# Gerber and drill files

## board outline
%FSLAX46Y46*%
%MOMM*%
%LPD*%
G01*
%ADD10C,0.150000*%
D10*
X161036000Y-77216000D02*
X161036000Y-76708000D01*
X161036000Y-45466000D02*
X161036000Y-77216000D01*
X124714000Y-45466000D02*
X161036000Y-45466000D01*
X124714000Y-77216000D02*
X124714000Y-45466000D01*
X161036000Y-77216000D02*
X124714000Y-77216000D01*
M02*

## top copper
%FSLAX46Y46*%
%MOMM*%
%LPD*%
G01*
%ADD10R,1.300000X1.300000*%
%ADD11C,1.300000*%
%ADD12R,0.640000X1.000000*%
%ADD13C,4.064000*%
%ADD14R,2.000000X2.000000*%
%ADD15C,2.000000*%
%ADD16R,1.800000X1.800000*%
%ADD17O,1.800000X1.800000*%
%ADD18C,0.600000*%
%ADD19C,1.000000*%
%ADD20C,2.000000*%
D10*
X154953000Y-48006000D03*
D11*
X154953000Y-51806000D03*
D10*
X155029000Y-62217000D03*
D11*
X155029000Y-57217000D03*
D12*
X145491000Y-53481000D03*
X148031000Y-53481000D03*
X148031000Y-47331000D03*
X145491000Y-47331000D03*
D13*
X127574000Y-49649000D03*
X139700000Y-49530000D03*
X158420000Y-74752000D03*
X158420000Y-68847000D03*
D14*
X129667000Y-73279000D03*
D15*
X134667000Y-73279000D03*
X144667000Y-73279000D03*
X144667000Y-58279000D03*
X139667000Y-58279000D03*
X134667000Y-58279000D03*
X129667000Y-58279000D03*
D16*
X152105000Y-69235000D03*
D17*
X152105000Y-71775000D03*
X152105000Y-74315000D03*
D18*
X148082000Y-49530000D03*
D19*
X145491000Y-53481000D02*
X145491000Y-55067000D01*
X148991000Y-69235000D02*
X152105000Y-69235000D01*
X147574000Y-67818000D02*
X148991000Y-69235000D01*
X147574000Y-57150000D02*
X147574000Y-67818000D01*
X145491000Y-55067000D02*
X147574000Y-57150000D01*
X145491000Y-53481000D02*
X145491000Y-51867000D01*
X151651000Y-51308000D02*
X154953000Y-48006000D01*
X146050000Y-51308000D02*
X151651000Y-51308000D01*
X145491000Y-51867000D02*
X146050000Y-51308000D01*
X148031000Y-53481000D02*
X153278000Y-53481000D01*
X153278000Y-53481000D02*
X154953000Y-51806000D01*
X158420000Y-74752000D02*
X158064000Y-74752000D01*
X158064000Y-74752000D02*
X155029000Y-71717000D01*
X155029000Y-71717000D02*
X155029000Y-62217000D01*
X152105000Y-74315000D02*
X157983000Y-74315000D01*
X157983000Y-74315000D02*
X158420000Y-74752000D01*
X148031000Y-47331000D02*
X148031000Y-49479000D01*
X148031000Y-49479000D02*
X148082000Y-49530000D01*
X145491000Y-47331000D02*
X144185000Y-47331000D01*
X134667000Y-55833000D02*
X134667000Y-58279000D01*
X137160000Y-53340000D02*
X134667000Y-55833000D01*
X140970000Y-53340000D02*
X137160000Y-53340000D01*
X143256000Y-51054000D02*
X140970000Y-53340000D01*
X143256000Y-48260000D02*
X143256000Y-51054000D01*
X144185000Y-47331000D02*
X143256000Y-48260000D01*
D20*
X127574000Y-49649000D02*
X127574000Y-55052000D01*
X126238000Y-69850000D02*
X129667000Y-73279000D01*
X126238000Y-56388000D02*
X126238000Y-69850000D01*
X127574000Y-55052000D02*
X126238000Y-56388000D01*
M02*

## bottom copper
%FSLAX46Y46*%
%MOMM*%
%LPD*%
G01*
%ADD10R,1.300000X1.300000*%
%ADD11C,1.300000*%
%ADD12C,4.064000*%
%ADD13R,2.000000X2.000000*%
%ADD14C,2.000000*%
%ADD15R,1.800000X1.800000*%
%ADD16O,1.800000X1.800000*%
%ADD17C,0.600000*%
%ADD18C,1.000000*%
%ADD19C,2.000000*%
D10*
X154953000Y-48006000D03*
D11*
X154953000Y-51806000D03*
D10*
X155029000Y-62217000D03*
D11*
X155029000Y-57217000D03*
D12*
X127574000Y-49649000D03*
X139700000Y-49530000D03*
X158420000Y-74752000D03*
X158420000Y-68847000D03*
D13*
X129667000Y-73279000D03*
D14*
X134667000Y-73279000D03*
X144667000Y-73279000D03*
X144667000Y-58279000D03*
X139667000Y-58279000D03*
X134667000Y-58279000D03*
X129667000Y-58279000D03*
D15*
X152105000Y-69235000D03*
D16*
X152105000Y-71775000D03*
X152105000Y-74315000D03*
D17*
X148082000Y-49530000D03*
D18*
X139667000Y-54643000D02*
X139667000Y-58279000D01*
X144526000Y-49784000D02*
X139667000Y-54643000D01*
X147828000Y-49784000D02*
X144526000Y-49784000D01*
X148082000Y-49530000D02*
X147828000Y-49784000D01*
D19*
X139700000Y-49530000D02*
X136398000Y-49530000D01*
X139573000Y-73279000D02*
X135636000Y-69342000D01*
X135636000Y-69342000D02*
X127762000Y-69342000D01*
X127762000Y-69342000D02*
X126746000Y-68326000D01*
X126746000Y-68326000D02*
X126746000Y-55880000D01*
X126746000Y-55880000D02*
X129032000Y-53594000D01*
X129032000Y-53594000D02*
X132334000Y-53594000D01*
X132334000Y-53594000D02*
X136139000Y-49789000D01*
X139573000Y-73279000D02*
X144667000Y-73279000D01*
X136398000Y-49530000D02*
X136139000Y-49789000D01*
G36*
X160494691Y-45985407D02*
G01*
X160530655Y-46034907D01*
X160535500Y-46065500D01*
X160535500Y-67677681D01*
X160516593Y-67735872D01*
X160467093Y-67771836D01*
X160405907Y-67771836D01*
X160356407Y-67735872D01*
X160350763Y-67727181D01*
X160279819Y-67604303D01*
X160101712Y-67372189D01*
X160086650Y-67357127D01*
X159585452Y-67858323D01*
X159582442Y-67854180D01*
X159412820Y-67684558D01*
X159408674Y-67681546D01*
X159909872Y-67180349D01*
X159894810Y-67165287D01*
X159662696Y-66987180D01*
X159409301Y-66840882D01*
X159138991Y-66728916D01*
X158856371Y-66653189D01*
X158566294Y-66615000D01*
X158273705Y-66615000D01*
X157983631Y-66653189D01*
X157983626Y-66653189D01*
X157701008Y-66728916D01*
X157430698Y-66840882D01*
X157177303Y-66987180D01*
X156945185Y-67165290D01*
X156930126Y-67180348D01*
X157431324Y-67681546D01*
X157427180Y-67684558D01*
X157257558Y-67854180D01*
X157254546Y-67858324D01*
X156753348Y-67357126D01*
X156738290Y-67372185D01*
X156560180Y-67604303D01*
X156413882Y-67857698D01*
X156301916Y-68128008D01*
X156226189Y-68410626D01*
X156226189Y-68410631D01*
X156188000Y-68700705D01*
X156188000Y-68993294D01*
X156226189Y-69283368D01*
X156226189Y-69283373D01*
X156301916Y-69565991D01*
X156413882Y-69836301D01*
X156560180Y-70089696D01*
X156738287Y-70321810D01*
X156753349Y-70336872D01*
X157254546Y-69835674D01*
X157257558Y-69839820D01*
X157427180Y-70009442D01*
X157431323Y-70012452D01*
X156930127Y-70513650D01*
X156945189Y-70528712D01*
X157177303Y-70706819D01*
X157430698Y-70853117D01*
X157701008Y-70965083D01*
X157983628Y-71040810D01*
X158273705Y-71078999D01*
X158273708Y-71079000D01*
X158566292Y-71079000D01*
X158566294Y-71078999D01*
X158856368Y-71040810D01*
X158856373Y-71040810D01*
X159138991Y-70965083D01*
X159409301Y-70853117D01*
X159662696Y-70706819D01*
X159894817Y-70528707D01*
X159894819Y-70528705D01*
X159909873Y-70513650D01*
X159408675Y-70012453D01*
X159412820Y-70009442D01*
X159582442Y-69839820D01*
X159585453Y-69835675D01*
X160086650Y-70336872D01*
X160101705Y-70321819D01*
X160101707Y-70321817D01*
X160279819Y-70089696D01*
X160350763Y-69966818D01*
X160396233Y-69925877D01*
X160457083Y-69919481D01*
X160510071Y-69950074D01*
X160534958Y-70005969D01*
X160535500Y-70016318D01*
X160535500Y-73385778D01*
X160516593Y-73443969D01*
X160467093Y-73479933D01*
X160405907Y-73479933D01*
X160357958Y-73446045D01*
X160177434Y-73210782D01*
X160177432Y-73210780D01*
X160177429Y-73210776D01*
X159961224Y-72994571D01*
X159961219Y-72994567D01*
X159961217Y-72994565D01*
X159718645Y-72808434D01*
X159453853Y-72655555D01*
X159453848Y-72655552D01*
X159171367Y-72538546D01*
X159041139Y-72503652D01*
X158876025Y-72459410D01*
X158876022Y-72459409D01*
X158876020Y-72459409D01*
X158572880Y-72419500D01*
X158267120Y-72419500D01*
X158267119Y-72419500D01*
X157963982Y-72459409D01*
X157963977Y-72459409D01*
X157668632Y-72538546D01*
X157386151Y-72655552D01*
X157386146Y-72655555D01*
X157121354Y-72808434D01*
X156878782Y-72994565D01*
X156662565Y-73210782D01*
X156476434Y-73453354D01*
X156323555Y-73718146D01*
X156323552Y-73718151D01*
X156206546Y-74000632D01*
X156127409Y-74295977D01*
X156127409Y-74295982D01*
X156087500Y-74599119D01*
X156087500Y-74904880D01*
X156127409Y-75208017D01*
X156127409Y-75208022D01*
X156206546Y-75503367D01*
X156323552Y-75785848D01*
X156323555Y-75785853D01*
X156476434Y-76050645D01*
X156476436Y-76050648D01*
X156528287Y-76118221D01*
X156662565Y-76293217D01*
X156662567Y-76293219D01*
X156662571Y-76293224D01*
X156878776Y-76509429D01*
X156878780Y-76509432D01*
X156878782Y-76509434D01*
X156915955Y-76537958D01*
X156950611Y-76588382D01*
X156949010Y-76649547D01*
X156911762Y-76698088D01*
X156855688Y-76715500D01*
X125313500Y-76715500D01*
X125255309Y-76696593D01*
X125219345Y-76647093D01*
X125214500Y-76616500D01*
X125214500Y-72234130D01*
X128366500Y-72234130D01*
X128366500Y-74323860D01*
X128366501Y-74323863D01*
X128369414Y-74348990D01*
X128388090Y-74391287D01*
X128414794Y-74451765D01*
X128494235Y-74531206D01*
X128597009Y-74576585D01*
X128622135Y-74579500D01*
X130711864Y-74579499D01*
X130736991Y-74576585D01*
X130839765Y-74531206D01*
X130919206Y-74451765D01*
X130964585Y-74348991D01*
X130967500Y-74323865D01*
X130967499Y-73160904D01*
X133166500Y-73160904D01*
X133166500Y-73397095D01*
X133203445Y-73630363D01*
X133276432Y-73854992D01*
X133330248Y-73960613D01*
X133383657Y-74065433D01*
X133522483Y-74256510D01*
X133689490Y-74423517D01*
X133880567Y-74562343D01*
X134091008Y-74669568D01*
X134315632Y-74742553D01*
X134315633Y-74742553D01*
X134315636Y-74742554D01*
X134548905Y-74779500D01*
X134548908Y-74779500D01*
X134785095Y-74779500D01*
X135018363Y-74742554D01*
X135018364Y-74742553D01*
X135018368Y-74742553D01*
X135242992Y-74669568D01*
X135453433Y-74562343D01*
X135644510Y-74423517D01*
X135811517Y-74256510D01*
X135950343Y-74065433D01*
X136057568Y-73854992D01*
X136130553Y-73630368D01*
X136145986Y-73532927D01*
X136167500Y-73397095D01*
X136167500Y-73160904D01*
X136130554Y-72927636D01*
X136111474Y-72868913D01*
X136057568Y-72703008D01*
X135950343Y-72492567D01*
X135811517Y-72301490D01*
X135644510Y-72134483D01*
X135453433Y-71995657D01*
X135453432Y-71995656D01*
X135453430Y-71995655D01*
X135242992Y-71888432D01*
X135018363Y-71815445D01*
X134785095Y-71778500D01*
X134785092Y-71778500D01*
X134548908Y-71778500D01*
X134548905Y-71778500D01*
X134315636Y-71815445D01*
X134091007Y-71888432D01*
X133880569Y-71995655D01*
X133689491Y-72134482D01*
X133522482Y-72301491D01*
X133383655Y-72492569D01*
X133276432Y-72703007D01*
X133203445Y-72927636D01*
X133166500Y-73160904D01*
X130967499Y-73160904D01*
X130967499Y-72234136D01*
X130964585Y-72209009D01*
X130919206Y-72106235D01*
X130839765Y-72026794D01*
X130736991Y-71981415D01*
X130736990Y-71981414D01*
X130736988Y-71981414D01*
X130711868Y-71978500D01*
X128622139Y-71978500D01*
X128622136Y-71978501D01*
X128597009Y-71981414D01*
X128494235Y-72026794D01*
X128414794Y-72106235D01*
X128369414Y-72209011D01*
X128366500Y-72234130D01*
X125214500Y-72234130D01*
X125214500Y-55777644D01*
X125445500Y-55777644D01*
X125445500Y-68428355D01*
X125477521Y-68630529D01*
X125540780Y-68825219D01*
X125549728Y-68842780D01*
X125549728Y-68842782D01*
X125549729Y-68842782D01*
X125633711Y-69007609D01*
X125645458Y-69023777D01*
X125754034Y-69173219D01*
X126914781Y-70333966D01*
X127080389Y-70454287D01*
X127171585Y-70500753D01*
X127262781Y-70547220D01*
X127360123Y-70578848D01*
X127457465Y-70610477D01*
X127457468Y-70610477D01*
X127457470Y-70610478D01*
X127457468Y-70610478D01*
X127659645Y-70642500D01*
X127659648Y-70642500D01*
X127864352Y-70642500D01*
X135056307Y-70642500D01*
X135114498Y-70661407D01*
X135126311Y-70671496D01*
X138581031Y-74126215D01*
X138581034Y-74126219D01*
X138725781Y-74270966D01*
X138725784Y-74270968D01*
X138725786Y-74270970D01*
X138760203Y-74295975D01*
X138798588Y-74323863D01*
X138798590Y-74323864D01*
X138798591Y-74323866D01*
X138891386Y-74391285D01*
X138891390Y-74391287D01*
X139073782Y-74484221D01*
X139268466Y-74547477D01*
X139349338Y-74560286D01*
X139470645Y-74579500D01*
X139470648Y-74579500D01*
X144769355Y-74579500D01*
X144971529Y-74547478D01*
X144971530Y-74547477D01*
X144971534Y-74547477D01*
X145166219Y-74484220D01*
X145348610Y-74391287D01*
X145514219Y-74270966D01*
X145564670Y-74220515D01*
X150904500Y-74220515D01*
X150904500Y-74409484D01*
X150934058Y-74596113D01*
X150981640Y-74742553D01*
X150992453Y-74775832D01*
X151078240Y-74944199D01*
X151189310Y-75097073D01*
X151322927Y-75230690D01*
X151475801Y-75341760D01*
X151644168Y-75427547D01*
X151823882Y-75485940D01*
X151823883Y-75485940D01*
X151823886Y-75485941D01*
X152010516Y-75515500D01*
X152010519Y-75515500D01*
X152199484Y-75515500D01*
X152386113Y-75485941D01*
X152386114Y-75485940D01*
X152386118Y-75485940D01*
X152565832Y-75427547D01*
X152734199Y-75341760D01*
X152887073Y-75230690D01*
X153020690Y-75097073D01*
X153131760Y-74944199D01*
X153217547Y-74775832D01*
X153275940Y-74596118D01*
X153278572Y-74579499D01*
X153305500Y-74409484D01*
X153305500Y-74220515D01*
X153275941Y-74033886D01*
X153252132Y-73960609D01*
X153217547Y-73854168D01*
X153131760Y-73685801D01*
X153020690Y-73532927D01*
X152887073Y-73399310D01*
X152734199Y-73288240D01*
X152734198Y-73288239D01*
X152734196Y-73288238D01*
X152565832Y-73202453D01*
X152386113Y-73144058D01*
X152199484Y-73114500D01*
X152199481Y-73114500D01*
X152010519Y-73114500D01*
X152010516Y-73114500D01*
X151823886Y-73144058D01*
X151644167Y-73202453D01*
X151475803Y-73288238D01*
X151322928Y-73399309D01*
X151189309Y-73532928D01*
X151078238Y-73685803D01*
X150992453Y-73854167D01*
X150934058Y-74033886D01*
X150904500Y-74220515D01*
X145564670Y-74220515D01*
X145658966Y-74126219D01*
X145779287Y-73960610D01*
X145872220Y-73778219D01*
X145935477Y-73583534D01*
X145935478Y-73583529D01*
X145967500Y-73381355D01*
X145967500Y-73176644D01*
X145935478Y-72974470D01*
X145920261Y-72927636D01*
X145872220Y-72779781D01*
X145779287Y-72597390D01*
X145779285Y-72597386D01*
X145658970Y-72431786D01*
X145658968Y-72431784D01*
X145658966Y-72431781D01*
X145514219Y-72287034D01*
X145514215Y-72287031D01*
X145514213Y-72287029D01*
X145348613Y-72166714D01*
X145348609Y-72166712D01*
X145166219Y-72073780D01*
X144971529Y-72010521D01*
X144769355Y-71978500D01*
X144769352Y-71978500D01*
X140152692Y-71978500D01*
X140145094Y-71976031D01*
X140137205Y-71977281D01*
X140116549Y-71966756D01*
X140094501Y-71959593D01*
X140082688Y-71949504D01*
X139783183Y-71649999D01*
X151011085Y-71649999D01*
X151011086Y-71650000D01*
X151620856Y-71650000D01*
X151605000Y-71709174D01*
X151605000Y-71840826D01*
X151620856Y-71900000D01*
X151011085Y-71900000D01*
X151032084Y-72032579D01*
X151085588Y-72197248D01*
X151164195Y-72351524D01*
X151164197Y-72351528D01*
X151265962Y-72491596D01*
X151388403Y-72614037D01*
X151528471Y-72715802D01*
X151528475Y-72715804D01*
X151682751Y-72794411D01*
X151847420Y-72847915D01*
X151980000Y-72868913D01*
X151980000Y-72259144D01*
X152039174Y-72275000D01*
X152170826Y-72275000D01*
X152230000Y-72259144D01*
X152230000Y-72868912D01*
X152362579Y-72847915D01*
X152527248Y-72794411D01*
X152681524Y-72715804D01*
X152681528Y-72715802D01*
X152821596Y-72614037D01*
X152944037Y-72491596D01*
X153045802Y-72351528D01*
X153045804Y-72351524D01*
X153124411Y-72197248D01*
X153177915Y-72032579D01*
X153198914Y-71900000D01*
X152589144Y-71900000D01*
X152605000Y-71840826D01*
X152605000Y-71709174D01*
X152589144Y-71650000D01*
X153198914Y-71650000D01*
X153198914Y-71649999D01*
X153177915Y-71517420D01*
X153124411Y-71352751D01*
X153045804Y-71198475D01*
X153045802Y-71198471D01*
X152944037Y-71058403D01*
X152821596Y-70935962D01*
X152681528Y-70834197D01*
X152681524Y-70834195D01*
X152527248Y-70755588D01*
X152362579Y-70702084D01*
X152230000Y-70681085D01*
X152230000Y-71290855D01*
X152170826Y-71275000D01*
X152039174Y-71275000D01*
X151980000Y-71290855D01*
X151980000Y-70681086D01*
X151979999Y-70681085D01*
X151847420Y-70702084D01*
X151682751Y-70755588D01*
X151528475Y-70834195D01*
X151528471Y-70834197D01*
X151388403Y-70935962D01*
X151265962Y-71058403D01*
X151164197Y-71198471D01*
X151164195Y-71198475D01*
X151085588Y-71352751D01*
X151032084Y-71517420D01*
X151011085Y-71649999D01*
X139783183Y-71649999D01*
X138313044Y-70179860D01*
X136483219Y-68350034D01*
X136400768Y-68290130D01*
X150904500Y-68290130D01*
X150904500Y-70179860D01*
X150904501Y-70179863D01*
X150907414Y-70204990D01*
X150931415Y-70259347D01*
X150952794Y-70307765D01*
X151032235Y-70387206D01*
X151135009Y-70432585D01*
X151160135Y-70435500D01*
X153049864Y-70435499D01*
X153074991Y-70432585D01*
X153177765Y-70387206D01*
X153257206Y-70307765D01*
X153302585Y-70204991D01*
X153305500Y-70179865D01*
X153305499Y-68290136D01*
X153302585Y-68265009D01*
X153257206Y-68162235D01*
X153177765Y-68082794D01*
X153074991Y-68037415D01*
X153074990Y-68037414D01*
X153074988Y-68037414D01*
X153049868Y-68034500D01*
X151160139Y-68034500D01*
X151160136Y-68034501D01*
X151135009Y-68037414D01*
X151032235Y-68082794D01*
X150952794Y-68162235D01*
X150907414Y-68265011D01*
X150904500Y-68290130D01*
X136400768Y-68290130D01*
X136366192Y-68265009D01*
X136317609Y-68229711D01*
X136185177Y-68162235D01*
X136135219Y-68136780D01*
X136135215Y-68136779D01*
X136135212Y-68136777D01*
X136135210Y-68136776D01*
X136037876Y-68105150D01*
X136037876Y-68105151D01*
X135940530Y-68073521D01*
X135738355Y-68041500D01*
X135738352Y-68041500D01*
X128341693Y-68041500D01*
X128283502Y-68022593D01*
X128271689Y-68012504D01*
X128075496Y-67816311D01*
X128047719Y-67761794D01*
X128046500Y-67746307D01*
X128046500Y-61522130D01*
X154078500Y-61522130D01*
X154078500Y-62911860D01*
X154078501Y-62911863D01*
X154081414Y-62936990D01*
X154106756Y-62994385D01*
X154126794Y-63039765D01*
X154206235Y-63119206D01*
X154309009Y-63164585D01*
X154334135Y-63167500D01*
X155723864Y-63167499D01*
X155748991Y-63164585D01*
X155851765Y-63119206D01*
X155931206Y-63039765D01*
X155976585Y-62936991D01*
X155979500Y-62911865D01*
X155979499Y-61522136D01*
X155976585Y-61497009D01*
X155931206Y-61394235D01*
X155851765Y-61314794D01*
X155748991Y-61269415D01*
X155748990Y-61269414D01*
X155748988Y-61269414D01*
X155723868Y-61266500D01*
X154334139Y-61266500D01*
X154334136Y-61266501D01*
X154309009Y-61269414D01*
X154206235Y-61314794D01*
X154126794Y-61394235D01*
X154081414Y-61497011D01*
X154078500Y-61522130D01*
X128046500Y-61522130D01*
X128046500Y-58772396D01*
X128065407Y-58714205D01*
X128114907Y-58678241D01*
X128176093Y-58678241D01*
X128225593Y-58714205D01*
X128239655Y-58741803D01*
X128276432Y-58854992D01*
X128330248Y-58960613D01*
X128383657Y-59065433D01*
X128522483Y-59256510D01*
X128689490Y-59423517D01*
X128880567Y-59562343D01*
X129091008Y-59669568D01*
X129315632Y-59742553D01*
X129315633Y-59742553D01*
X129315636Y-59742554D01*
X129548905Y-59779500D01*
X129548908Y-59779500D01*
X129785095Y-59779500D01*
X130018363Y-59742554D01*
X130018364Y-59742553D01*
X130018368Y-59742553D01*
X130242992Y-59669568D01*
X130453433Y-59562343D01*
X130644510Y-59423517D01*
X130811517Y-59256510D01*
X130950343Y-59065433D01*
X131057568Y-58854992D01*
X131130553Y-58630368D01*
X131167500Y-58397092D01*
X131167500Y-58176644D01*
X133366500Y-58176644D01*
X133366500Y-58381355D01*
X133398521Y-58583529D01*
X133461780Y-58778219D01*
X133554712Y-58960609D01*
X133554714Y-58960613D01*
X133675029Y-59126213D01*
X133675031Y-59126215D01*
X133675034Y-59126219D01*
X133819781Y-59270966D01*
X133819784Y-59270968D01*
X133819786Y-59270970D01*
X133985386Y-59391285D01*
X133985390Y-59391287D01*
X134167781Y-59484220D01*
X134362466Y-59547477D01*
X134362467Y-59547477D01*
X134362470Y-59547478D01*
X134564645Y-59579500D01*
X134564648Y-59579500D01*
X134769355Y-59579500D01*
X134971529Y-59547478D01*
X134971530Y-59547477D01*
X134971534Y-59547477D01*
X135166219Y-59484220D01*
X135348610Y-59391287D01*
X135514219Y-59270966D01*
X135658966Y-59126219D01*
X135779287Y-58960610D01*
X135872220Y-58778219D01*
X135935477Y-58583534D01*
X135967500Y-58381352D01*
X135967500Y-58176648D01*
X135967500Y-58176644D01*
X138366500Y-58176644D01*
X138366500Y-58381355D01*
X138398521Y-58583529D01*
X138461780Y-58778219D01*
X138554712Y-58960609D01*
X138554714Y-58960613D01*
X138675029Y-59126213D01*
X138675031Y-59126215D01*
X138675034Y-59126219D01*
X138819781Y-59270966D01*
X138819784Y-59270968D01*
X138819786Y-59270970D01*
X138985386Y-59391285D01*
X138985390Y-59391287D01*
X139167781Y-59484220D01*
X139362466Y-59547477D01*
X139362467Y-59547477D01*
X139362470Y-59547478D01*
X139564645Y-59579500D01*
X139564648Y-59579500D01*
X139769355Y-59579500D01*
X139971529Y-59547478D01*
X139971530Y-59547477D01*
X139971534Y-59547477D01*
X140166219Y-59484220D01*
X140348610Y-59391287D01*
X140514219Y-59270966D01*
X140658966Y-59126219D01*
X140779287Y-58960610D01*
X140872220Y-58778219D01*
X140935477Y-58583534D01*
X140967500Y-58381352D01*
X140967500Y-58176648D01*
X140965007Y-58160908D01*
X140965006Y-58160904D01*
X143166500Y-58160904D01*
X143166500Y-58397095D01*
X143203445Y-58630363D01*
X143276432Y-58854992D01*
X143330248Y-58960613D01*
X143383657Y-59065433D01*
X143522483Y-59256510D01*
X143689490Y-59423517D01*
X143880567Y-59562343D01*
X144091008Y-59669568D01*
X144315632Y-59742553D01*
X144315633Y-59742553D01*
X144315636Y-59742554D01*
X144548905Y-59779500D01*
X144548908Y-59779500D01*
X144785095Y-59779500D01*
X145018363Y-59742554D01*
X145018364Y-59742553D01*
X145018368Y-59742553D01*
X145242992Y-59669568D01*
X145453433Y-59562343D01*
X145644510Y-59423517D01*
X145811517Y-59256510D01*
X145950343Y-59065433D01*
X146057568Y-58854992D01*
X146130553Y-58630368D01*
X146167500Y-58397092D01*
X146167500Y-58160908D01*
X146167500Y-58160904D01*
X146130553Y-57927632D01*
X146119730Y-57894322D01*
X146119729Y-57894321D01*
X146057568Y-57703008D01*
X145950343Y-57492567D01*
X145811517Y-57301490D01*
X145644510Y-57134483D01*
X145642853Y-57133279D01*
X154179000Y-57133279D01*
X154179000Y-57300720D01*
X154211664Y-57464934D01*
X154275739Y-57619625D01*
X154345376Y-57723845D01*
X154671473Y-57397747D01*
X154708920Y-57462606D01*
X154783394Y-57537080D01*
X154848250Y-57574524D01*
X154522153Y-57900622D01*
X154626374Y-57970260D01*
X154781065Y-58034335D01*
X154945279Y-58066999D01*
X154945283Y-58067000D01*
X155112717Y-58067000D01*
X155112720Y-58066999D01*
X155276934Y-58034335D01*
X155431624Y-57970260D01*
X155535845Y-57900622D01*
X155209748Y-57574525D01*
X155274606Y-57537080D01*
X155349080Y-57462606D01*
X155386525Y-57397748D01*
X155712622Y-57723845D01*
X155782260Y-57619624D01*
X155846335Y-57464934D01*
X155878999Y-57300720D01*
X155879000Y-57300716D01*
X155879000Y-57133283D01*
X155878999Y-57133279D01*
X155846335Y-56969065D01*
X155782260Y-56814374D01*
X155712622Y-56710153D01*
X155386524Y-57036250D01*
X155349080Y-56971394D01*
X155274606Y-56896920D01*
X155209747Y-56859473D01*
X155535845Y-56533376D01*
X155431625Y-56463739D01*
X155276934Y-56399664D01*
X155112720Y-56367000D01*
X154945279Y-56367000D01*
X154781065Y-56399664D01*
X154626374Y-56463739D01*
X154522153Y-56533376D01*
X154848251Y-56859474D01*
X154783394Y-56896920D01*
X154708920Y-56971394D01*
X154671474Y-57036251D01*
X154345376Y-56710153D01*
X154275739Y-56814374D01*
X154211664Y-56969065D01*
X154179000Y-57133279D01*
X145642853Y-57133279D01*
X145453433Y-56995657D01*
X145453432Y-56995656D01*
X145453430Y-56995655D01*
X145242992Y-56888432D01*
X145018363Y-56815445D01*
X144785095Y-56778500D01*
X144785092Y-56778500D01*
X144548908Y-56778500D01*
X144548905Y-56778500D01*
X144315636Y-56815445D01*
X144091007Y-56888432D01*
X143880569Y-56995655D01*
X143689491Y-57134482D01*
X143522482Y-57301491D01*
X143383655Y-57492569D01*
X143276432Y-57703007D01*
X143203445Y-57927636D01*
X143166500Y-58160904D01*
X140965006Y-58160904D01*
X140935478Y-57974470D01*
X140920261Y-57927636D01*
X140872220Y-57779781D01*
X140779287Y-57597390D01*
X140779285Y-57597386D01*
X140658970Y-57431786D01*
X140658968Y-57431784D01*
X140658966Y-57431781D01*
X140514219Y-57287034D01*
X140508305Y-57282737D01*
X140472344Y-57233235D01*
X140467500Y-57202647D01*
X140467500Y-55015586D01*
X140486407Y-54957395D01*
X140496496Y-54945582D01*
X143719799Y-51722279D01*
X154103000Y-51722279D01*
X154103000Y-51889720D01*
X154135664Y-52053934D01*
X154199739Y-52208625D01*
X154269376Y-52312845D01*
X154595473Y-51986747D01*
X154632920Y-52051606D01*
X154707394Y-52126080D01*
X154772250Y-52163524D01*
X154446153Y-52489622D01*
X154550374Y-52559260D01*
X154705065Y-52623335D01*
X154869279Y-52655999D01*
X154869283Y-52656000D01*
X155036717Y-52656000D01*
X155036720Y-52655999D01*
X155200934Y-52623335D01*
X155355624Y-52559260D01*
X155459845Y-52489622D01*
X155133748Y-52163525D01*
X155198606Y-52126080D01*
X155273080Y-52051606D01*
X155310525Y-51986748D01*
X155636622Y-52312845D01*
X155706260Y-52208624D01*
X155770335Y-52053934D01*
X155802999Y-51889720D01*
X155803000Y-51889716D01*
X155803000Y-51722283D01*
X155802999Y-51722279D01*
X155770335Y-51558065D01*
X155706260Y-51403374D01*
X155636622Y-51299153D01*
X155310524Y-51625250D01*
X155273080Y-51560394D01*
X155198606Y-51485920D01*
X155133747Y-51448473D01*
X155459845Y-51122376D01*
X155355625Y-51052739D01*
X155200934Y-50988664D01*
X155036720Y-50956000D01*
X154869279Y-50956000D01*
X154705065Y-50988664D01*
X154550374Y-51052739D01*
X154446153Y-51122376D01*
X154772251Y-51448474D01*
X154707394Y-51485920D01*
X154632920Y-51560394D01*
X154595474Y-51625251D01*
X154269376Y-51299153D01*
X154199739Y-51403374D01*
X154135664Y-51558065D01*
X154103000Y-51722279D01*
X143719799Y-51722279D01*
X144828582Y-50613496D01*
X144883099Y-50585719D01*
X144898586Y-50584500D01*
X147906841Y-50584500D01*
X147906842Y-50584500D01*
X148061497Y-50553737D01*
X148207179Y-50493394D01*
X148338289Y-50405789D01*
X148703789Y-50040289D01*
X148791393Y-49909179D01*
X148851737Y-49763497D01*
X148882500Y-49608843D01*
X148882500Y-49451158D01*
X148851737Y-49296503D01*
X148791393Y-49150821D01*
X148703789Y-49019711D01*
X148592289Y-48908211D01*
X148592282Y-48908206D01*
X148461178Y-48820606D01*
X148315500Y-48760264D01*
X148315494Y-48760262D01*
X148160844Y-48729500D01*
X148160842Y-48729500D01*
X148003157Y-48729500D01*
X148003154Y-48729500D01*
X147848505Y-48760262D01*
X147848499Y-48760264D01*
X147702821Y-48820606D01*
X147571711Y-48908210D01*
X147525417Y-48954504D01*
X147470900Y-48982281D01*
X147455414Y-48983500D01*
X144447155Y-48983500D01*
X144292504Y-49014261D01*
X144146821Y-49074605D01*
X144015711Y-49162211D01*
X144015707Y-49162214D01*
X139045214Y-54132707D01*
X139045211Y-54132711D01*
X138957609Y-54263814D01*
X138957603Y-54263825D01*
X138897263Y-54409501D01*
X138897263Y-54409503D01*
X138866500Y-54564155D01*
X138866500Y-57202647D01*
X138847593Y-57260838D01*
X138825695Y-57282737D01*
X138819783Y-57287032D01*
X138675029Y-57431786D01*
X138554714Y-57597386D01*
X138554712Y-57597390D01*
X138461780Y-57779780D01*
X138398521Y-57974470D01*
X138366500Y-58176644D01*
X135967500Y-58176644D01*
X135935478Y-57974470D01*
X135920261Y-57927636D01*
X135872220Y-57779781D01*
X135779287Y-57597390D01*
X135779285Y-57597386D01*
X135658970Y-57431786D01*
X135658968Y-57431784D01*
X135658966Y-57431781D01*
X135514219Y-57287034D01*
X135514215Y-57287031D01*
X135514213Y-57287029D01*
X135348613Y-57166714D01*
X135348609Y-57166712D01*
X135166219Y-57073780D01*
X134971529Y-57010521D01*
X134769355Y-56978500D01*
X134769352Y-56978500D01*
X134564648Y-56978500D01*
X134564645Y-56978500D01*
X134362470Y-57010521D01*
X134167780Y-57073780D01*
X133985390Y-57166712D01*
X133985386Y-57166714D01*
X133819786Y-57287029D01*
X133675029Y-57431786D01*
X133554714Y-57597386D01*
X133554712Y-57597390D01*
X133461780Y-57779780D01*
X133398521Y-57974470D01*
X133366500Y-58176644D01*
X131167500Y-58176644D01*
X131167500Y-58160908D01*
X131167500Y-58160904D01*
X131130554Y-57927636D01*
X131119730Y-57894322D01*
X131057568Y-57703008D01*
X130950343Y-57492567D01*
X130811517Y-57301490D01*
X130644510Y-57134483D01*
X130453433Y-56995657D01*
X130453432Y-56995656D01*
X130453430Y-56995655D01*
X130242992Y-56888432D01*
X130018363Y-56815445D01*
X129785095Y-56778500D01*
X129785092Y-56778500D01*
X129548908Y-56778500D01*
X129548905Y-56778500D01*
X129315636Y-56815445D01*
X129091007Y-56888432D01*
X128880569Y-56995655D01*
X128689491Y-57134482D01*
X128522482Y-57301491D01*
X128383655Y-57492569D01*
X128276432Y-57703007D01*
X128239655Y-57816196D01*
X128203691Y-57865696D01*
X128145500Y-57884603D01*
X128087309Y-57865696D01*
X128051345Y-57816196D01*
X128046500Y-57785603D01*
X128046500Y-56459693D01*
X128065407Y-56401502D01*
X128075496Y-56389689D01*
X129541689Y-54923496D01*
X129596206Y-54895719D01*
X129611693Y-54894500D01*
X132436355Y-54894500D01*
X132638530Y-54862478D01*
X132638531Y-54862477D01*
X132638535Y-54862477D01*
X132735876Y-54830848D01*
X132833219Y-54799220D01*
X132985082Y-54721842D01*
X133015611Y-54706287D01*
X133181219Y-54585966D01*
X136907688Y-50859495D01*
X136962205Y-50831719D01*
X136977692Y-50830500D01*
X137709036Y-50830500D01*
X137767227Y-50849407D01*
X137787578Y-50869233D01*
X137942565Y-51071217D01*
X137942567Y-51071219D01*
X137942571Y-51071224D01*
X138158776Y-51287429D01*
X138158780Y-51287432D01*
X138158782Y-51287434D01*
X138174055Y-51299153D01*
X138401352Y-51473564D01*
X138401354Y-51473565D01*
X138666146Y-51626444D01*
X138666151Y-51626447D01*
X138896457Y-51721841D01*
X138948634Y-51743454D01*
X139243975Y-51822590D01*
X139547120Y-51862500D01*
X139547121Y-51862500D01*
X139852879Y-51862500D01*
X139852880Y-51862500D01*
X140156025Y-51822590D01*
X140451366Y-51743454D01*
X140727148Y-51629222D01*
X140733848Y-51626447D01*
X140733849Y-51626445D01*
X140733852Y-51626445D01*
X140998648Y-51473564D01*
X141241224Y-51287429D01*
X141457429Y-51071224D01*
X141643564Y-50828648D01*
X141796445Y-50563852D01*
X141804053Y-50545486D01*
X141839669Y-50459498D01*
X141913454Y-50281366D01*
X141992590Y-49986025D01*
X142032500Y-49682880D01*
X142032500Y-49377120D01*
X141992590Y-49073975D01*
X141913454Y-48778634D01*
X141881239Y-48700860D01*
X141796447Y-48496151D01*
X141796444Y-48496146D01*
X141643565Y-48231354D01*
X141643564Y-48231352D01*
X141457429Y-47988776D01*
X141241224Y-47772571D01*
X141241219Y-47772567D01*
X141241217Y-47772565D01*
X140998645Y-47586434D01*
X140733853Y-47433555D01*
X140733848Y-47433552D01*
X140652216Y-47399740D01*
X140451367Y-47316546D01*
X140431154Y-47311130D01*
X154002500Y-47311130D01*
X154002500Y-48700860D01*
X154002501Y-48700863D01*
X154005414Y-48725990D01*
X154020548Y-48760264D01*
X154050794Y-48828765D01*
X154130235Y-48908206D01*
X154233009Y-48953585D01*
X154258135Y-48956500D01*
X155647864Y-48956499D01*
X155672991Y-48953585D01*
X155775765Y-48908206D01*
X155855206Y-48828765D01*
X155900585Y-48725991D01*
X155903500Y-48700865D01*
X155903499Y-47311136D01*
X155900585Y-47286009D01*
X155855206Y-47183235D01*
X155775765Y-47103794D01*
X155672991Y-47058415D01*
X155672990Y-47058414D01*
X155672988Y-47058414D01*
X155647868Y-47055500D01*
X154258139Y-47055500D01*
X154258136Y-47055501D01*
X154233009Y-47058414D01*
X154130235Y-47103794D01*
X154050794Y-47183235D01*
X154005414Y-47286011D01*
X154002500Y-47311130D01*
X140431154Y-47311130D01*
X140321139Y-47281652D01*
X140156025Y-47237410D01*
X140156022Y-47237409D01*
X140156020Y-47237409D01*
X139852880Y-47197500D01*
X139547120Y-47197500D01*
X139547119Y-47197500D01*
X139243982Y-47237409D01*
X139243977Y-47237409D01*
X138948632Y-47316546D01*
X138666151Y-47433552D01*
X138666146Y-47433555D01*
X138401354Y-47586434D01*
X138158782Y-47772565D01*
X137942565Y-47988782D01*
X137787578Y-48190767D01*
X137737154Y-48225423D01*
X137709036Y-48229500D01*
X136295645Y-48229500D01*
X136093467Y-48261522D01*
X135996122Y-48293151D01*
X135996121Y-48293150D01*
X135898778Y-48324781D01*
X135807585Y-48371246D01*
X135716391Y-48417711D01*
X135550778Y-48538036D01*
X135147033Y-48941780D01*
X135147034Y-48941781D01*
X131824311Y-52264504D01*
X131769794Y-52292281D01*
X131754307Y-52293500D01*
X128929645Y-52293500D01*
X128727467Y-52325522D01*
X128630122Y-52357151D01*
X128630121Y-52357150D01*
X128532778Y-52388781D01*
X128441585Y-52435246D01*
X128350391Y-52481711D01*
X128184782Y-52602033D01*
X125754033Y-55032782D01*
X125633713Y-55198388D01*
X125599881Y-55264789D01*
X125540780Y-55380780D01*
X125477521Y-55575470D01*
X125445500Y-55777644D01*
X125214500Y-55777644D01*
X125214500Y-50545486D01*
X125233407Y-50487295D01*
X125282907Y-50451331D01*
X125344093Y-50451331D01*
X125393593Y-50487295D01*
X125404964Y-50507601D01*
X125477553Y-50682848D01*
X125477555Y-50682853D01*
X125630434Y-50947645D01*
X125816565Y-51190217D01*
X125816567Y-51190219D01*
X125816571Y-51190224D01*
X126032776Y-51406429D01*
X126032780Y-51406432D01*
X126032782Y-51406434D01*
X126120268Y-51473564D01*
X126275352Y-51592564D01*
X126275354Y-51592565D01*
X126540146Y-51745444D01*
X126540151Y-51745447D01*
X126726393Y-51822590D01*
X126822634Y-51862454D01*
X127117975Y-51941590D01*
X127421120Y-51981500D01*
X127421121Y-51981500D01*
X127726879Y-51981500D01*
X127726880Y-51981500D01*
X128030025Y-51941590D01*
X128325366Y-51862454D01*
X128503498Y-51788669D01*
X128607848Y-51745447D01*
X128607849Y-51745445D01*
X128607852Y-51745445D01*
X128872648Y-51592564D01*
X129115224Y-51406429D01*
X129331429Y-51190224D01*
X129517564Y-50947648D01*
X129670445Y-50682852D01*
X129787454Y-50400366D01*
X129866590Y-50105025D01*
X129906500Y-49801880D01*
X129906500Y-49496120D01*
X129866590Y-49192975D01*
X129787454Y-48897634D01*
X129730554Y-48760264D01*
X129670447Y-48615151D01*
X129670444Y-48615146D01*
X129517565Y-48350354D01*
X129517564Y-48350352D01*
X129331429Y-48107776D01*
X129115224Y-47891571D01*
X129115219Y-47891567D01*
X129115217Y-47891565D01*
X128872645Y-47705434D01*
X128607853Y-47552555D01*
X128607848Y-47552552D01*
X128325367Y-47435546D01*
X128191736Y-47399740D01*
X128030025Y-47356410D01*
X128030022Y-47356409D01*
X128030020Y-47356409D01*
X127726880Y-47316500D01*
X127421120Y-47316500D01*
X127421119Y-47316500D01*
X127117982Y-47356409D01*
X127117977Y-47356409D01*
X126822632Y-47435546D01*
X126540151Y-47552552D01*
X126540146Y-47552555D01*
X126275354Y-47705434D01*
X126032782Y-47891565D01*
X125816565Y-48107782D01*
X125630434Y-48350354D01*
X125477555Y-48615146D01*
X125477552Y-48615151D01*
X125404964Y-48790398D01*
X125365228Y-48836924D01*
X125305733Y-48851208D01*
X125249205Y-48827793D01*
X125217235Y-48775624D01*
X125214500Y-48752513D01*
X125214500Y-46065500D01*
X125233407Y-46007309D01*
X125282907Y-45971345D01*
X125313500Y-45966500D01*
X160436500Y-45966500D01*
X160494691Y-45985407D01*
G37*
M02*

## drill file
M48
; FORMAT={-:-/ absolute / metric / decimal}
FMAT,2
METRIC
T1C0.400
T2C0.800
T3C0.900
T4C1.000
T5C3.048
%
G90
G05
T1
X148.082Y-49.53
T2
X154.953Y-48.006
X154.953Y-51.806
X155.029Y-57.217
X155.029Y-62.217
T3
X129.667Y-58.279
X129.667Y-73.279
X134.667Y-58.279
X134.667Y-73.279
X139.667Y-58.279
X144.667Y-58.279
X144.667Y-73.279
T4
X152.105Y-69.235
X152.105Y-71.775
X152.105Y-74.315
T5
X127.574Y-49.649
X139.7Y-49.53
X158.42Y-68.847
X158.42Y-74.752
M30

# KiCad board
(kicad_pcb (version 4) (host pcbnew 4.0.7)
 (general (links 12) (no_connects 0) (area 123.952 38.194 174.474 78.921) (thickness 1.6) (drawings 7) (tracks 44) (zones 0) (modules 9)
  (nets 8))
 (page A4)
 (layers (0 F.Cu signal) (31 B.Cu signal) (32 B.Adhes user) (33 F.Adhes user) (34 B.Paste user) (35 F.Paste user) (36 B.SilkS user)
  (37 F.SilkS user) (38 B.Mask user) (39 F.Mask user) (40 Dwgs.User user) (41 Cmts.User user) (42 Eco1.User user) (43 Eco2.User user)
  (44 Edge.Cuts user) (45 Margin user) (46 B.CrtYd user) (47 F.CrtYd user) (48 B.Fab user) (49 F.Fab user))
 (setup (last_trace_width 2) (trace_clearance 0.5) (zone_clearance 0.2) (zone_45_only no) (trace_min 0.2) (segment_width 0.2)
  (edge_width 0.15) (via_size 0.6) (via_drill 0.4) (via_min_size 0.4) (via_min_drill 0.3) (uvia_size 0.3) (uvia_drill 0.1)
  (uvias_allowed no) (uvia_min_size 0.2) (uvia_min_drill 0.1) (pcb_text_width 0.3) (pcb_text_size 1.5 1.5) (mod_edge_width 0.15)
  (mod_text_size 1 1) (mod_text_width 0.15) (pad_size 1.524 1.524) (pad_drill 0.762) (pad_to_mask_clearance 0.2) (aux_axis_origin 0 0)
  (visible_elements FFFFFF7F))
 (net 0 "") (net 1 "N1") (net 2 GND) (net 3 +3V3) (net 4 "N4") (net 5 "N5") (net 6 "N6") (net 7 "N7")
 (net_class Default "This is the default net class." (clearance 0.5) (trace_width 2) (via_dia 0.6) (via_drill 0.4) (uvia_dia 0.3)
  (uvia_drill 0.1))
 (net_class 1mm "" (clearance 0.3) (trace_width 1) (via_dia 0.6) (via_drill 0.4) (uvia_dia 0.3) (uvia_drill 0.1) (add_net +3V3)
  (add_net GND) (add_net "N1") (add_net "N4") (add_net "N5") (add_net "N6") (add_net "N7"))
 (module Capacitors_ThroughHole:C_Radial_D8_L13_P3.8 (layer F.Cu) (at 154.953 48.006 270)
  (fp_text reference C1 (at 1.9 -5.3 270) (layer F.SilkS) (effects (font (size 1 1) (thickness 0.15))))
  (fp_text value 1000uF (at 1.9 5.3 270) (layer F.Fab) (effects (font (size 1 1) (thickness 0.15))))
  (pad 1 thru_hole rect (at 0 0 270) (size 1.3 1.3) (drill 0.8) (layers *.Cu *.Mask) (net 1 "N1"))
  (pad 2 thru_hole circle (at 3.8 0 270) (size 1.3 1.3) (drill 0.8) (layers *.Cu *.Mask) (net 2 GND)))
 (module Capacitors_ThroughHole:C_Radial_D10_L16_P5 (layer F.Cu) (at 155.029 62.217 90)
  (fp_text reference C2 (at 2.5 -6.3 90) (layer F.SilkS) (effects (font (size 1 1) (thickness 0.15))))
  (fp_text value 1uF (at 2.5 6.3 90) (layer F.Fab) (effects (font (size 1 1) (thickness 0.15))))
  (pad 1 thru_hole rect (at 0 0 90) (size 1.3 1.3) (drill 0.8) (layers *.Cu *.Mask) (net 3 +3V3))
  (pad 2 thru_hole circle (at 5 0 90) (size 1.3 1.3) (drill 0.8) (layers *.Cu *.Mask) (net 2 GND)))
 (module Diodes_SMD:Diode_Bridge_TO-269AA (layer F.Cu) (at 146.761 50.406 90)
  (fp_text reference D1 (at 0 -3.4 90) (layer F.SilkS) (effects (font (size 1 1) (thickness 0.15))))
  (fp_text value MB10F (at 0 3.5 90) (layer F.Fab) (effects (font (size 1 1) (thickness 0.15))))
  (pad 1 smd rect (at -3.075 -1.27 90) (size 1 0.64) (layers F.Cu F.Paste F.Mask) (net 1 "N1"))
  (pad 2 smd rect (at -3.075 1.27 90) (size 1 0.64) (layers F.Cu F.Paste F.Mask) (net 2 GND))
  (pad 3 smd rect (at 3.075 1.27 90) (size 1 0.64) (layers F.Cu F.Paste F.Mask) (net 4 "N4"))
  (pad 4 smd rect (at 3.075 -1.27 90) (size 1 0.64) (layers F.Cu F.Paste F.Mask) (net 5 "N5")))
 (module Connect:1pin (layer F.Cu) (at 127.574 49.649)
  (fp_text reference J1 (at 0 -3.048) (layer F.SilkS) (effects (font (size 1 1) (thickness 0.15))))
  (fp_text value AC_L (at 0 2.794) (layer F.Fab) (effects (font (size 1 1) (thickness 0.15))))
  (pad 1 thru_hole circle (at 0 0) (size 4.064 4.064) (drill 3.048) (layers *.Cu *.Mask) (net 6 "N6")))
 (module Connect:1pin (layer F.Cu) (at 139.7 49.53)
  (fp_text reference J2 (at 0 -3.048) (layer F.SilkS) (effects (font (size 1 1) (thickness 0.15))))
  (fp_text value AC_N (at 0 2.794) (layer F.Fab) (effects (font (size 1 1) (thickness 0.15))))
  (pad 1 thru_hole circle (at 0 0) (size 4.064 4.064) (drill 3.048) (layers *.Cu *.Mask) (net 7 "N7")))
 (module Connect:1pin (layer F.Cu) (at 158.42 74.752)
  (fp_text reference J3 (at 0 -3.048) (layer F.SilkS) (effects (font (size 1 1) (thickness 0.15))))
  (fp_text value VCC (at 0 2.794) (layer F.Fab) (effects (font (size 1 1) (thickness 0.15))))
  (pad 1 thru_hole circle (at 0 0) (size 4.064 4.064) (drill 3.048) (layers *.Cu *.Mask) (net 3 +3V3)))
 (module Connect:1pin (layer F.Cu) (at 158.42 68.847)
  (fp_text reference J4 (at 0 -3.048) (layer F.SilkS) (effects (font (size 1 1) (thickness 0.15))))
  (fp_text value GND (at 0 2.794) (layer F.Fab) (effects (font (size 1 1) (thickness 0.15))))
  (pad 1 thru_hole circle (at 0 0) (size 4.064 4.064) (drill 3.048) (layers *.Cu *.Mask) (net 2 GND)))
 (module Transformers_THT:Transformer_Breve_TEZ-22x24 (layer F.Cu) (at 129.667 73.279)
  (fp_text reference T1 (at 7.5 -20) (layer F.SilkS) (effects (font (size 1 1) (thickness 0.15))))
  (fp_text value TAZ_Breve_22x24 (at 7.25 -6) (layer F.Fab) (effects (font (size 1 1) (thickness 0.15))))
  (pad 1 thru_hole rect (at 0 0) (size 2 2) (drill 0.9) (layers *.Cu *.Mask) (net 6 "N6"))
  (pad 2 thru_hole circle (at 5 0) (size 2 2) (drill 0.9) (layers *.Cu *.Mask))
  (pad 4 thru_hole circle (at 15 0) (size 2 2) (drill 0.9) (layers *.Cu *.Mask) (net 7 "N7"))
  (pad 5 thru_hole circle (at 15 -15) (size 2 2) (drill 0.9) (layers *.Cu *.Mask))
  (pad 6 thru_hole circle (at 10 -15) (size 2 2) (drill 0.9) (layers *.Cu *.Mask) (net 4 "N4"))
  (pad 7 thru_hole circle (at 5 -15) (size 2 2) (drill 0.9) (layers *.Cu *.Mask) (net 5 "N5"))
  (pad 8 thru_hole circle (at 0 -15) (size 2 2) (drill 0.9) (layers *.Cu *.Mask)))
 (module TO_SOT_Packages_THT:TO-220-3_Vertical (layer F.Cu) (at 152.105 69.235 270)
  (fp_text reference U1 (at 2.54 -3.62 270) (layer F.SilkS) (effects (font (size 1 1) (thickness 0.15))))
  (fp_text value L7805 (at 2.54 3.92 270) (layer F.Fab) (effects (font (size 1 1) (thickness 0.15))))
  (pad 1 thru_hole rect (at 0 0 270) (size 1.8 1.8) (drill 1) (layers *.Cu *.Mask) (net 1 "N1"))
  (pad 2 thru_hole oval (at 2.54 0 270) (size 1.8 1.8) (drill 1) (layers *.Cu *.Mask) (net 2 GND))
  (pad 3 thru_hole oval (at 5.08 0 270) (size 1.8 1.8) (drill 1) (layers *.Cu *.Mask) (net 3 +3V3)))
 (gr_line (start 161.036 77.216) (end 161.036 76.708) (angle 90) (layer Edge.Cuts) (width 0.15))
 (gr_line (start 161.036 45.466) (end 161.036 77.216) (angle 90) (layer Edge.Cuts) (width 0.15))
 (gr_line (start 124.714 45.466) (end 161.036 45.466) (angle 90) (layer Edge.Cuts) (width 0.15))
 (gr_line (start 124.714 77.216) (end 124.714 45.466) (angle 90) (layer Edge.Cuts) (width 0.15))
 (gr_line (start 161.036 77.216) (end 124.714 77.216) (angle 90) (layer Edge.Cuts) (width 0.15))
 (segment (start 145.491 53.481) (end 145.491 55.067) (width 1) (layer F.Cu) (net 1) (status 400000))
 (segment (start 148.991 69.235) (end 152.105 69.235) (width 1) (layer F.Cu) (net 1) (status 800000))
 (segment (start 147.574 67.818) (end 148.991 69.235) (width 1) (layer F.Cu) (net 1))
 (segment (start 147.574 57.15) (end 147.574 67.818) (width 1) (layer F.Cu) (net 1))
 (segment (start 145.491 55.067) (end 147.574 57.15) (width 1) (layer F.Cu) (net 1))
 (segment (start 145.491 53.481) (end 145.491 51.867) (width 1) (layer F.Cu) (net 1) (status 400000))
 (segment (start 151.651 51.308) (end 154.953 48.006) (width 1) (layer F.Cu) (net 1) (status 800000))
 (segment (start 146.05 51.308) (end 151.651 51.308) (width 1) (layer F.Cu) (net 1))
 (segment (start 145.491 51.867) (end 146.05 51.308) (width 1) (layer F.Cu) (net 1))
 (segment (start 148.031 53.481) (end 153.278 53.481) (width 1) (layer F.Cu) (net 2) (status 400000))
 (segment (start 153.278 53.481) (end 154.953 51.806) (width 1) (layer F.Cu) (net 2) (status 800000))
 (segment (start 158.42 74.752) (end 158.064 74.752) (width 1) (layer F.Cu) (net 3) (status C00000))
 (segment (start 158.064 74.752) (end 155.029 71.717) (width 1) (layer F.Cu) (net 3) (status 400000))
 (segment (start 155.029 71.717) (end 155.029 62.217) (width 1) (layer F.Cu) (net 3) (status 800000))
 (segment (start 152.105 74.315) (end 157.983 74.315) (width 1) (layer F.Cu) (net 3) (status C00000))
 (segment (start 157.983 74.315) (end 158.42 74.752) (width 1) (layer F.Cu) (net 3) (status C00000))
 (segment (start 148.031 47.331) (end 148.031 49.479) (width 1) (layer F.Cu) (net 4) (status 400000))
 (segment (start 139.667 54.643) (end 139.667 58.279) (width 1) (layer B.Cu) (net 4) (status 800000))
 (segment (start 144.526 49.784) (end 139.667 54.643) (width 1) (layer B.Cu) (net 4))
 (segment (start 147.828 49.784) (end 144.526 49.784) (width 1) (layer B.Cu) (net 4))
 (segment (start 148.082 49.53) (end 147.828 49.784) (width 1) (layer B.Cu) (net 4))
 (via (at 148.082 49.53) (size 0.6) (drill 0.4) (layers F.Cu B.Cu) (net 4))
 (segment (start 148.031 49.479) (end 148.082 49.53) (width 1) (layer F.Cu) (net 4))
 (segment (start 145.491 47.331) (end 144.185 47.331) (width 1) (layer F.Cu) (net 5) (status 400000))
 (segment (start 134.667 55.833) (end 134.667 58.279) (width 1) (layer F.Cu) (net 5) (status 800000))
 (segment (start 137.16 53.34) (end 134.667 55.833) (width 1) (layer F.Cu) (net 5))
 (segment (start 140.97 53.34) (end 137.16 53.34) (width 1) (layer F.Cu) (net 5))
 (segment (start 143.256 51.054) (end 140.97 53.34) (width 1) (layer F.Cu) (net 5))
 (segment (start 143.256 48.26) (end 143.256 51.054) (width 1) (layer F.Cu) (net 5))
 (segment (start 144.185 47.331) (end 143.256 48.26) (width 1) (layer F.Cu) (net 5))
 (segment (start 127.574 49.649) (end 127.574 55.052) (width 2) (layer F.Cu) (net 6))
 (segment (start 126.238 69.85) (end 129.667 73.279) (width 2) (layer F.Cu) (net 6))
 (segment (start 126.238 56.388) (end 126.238 69.85) (width 2) (layer F.Cu) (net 6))
 (segment (start 127.574 55.052) (end 126.238 56.388) (width 2) (layer F.Cu) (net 6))
 (segment (start 139.7 49.53) (end 136.398 49.53) (width 2) (layer B.Cu) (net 7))
 (segment (start 139.573 73.279) (end 135.636 69.342) (width 2) (layer B.Cu) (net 7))
 (segment (start 135.636 69.342) (end 127.762 69.342) (width 2) (layer B.Cu) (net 7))
 (segment (start 127.762 69.342) (end 126.746 68.326) (width 2) (layer B.Cu) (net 7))
 (segment (start 126.746 68.326) (end 126.746 55.88) (width 2) (layer B.Cu) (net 7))
 (segment (start 126.746 55.88) (end 129.032 53.594) (width 2) (layer B.Cu) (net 7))
 (segment (start 129.032 53.594) (end 132.334 53.594) (width 2) (layer B.Cu) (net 7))
 (segment (start 132.334 53.594) (end 136.139 49.789) (width 2) (layer B.Cu) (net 7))
 (segment (start 139.573 73.279) (end 144.667 73.279) (width 2) (layer B.Cu) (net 7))
 (segment (start 136.398 49.53) (end 136.139 49.789) (width 2) (layer B.Cu) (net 7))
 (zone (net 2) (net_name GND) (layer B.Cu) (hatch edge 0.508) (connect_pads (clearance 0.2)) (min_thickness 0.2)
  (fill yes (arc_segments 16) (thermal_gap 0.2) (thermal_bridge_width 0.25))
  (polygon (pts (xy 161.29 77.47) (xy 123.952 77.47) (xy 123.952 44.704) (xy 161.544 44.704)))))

